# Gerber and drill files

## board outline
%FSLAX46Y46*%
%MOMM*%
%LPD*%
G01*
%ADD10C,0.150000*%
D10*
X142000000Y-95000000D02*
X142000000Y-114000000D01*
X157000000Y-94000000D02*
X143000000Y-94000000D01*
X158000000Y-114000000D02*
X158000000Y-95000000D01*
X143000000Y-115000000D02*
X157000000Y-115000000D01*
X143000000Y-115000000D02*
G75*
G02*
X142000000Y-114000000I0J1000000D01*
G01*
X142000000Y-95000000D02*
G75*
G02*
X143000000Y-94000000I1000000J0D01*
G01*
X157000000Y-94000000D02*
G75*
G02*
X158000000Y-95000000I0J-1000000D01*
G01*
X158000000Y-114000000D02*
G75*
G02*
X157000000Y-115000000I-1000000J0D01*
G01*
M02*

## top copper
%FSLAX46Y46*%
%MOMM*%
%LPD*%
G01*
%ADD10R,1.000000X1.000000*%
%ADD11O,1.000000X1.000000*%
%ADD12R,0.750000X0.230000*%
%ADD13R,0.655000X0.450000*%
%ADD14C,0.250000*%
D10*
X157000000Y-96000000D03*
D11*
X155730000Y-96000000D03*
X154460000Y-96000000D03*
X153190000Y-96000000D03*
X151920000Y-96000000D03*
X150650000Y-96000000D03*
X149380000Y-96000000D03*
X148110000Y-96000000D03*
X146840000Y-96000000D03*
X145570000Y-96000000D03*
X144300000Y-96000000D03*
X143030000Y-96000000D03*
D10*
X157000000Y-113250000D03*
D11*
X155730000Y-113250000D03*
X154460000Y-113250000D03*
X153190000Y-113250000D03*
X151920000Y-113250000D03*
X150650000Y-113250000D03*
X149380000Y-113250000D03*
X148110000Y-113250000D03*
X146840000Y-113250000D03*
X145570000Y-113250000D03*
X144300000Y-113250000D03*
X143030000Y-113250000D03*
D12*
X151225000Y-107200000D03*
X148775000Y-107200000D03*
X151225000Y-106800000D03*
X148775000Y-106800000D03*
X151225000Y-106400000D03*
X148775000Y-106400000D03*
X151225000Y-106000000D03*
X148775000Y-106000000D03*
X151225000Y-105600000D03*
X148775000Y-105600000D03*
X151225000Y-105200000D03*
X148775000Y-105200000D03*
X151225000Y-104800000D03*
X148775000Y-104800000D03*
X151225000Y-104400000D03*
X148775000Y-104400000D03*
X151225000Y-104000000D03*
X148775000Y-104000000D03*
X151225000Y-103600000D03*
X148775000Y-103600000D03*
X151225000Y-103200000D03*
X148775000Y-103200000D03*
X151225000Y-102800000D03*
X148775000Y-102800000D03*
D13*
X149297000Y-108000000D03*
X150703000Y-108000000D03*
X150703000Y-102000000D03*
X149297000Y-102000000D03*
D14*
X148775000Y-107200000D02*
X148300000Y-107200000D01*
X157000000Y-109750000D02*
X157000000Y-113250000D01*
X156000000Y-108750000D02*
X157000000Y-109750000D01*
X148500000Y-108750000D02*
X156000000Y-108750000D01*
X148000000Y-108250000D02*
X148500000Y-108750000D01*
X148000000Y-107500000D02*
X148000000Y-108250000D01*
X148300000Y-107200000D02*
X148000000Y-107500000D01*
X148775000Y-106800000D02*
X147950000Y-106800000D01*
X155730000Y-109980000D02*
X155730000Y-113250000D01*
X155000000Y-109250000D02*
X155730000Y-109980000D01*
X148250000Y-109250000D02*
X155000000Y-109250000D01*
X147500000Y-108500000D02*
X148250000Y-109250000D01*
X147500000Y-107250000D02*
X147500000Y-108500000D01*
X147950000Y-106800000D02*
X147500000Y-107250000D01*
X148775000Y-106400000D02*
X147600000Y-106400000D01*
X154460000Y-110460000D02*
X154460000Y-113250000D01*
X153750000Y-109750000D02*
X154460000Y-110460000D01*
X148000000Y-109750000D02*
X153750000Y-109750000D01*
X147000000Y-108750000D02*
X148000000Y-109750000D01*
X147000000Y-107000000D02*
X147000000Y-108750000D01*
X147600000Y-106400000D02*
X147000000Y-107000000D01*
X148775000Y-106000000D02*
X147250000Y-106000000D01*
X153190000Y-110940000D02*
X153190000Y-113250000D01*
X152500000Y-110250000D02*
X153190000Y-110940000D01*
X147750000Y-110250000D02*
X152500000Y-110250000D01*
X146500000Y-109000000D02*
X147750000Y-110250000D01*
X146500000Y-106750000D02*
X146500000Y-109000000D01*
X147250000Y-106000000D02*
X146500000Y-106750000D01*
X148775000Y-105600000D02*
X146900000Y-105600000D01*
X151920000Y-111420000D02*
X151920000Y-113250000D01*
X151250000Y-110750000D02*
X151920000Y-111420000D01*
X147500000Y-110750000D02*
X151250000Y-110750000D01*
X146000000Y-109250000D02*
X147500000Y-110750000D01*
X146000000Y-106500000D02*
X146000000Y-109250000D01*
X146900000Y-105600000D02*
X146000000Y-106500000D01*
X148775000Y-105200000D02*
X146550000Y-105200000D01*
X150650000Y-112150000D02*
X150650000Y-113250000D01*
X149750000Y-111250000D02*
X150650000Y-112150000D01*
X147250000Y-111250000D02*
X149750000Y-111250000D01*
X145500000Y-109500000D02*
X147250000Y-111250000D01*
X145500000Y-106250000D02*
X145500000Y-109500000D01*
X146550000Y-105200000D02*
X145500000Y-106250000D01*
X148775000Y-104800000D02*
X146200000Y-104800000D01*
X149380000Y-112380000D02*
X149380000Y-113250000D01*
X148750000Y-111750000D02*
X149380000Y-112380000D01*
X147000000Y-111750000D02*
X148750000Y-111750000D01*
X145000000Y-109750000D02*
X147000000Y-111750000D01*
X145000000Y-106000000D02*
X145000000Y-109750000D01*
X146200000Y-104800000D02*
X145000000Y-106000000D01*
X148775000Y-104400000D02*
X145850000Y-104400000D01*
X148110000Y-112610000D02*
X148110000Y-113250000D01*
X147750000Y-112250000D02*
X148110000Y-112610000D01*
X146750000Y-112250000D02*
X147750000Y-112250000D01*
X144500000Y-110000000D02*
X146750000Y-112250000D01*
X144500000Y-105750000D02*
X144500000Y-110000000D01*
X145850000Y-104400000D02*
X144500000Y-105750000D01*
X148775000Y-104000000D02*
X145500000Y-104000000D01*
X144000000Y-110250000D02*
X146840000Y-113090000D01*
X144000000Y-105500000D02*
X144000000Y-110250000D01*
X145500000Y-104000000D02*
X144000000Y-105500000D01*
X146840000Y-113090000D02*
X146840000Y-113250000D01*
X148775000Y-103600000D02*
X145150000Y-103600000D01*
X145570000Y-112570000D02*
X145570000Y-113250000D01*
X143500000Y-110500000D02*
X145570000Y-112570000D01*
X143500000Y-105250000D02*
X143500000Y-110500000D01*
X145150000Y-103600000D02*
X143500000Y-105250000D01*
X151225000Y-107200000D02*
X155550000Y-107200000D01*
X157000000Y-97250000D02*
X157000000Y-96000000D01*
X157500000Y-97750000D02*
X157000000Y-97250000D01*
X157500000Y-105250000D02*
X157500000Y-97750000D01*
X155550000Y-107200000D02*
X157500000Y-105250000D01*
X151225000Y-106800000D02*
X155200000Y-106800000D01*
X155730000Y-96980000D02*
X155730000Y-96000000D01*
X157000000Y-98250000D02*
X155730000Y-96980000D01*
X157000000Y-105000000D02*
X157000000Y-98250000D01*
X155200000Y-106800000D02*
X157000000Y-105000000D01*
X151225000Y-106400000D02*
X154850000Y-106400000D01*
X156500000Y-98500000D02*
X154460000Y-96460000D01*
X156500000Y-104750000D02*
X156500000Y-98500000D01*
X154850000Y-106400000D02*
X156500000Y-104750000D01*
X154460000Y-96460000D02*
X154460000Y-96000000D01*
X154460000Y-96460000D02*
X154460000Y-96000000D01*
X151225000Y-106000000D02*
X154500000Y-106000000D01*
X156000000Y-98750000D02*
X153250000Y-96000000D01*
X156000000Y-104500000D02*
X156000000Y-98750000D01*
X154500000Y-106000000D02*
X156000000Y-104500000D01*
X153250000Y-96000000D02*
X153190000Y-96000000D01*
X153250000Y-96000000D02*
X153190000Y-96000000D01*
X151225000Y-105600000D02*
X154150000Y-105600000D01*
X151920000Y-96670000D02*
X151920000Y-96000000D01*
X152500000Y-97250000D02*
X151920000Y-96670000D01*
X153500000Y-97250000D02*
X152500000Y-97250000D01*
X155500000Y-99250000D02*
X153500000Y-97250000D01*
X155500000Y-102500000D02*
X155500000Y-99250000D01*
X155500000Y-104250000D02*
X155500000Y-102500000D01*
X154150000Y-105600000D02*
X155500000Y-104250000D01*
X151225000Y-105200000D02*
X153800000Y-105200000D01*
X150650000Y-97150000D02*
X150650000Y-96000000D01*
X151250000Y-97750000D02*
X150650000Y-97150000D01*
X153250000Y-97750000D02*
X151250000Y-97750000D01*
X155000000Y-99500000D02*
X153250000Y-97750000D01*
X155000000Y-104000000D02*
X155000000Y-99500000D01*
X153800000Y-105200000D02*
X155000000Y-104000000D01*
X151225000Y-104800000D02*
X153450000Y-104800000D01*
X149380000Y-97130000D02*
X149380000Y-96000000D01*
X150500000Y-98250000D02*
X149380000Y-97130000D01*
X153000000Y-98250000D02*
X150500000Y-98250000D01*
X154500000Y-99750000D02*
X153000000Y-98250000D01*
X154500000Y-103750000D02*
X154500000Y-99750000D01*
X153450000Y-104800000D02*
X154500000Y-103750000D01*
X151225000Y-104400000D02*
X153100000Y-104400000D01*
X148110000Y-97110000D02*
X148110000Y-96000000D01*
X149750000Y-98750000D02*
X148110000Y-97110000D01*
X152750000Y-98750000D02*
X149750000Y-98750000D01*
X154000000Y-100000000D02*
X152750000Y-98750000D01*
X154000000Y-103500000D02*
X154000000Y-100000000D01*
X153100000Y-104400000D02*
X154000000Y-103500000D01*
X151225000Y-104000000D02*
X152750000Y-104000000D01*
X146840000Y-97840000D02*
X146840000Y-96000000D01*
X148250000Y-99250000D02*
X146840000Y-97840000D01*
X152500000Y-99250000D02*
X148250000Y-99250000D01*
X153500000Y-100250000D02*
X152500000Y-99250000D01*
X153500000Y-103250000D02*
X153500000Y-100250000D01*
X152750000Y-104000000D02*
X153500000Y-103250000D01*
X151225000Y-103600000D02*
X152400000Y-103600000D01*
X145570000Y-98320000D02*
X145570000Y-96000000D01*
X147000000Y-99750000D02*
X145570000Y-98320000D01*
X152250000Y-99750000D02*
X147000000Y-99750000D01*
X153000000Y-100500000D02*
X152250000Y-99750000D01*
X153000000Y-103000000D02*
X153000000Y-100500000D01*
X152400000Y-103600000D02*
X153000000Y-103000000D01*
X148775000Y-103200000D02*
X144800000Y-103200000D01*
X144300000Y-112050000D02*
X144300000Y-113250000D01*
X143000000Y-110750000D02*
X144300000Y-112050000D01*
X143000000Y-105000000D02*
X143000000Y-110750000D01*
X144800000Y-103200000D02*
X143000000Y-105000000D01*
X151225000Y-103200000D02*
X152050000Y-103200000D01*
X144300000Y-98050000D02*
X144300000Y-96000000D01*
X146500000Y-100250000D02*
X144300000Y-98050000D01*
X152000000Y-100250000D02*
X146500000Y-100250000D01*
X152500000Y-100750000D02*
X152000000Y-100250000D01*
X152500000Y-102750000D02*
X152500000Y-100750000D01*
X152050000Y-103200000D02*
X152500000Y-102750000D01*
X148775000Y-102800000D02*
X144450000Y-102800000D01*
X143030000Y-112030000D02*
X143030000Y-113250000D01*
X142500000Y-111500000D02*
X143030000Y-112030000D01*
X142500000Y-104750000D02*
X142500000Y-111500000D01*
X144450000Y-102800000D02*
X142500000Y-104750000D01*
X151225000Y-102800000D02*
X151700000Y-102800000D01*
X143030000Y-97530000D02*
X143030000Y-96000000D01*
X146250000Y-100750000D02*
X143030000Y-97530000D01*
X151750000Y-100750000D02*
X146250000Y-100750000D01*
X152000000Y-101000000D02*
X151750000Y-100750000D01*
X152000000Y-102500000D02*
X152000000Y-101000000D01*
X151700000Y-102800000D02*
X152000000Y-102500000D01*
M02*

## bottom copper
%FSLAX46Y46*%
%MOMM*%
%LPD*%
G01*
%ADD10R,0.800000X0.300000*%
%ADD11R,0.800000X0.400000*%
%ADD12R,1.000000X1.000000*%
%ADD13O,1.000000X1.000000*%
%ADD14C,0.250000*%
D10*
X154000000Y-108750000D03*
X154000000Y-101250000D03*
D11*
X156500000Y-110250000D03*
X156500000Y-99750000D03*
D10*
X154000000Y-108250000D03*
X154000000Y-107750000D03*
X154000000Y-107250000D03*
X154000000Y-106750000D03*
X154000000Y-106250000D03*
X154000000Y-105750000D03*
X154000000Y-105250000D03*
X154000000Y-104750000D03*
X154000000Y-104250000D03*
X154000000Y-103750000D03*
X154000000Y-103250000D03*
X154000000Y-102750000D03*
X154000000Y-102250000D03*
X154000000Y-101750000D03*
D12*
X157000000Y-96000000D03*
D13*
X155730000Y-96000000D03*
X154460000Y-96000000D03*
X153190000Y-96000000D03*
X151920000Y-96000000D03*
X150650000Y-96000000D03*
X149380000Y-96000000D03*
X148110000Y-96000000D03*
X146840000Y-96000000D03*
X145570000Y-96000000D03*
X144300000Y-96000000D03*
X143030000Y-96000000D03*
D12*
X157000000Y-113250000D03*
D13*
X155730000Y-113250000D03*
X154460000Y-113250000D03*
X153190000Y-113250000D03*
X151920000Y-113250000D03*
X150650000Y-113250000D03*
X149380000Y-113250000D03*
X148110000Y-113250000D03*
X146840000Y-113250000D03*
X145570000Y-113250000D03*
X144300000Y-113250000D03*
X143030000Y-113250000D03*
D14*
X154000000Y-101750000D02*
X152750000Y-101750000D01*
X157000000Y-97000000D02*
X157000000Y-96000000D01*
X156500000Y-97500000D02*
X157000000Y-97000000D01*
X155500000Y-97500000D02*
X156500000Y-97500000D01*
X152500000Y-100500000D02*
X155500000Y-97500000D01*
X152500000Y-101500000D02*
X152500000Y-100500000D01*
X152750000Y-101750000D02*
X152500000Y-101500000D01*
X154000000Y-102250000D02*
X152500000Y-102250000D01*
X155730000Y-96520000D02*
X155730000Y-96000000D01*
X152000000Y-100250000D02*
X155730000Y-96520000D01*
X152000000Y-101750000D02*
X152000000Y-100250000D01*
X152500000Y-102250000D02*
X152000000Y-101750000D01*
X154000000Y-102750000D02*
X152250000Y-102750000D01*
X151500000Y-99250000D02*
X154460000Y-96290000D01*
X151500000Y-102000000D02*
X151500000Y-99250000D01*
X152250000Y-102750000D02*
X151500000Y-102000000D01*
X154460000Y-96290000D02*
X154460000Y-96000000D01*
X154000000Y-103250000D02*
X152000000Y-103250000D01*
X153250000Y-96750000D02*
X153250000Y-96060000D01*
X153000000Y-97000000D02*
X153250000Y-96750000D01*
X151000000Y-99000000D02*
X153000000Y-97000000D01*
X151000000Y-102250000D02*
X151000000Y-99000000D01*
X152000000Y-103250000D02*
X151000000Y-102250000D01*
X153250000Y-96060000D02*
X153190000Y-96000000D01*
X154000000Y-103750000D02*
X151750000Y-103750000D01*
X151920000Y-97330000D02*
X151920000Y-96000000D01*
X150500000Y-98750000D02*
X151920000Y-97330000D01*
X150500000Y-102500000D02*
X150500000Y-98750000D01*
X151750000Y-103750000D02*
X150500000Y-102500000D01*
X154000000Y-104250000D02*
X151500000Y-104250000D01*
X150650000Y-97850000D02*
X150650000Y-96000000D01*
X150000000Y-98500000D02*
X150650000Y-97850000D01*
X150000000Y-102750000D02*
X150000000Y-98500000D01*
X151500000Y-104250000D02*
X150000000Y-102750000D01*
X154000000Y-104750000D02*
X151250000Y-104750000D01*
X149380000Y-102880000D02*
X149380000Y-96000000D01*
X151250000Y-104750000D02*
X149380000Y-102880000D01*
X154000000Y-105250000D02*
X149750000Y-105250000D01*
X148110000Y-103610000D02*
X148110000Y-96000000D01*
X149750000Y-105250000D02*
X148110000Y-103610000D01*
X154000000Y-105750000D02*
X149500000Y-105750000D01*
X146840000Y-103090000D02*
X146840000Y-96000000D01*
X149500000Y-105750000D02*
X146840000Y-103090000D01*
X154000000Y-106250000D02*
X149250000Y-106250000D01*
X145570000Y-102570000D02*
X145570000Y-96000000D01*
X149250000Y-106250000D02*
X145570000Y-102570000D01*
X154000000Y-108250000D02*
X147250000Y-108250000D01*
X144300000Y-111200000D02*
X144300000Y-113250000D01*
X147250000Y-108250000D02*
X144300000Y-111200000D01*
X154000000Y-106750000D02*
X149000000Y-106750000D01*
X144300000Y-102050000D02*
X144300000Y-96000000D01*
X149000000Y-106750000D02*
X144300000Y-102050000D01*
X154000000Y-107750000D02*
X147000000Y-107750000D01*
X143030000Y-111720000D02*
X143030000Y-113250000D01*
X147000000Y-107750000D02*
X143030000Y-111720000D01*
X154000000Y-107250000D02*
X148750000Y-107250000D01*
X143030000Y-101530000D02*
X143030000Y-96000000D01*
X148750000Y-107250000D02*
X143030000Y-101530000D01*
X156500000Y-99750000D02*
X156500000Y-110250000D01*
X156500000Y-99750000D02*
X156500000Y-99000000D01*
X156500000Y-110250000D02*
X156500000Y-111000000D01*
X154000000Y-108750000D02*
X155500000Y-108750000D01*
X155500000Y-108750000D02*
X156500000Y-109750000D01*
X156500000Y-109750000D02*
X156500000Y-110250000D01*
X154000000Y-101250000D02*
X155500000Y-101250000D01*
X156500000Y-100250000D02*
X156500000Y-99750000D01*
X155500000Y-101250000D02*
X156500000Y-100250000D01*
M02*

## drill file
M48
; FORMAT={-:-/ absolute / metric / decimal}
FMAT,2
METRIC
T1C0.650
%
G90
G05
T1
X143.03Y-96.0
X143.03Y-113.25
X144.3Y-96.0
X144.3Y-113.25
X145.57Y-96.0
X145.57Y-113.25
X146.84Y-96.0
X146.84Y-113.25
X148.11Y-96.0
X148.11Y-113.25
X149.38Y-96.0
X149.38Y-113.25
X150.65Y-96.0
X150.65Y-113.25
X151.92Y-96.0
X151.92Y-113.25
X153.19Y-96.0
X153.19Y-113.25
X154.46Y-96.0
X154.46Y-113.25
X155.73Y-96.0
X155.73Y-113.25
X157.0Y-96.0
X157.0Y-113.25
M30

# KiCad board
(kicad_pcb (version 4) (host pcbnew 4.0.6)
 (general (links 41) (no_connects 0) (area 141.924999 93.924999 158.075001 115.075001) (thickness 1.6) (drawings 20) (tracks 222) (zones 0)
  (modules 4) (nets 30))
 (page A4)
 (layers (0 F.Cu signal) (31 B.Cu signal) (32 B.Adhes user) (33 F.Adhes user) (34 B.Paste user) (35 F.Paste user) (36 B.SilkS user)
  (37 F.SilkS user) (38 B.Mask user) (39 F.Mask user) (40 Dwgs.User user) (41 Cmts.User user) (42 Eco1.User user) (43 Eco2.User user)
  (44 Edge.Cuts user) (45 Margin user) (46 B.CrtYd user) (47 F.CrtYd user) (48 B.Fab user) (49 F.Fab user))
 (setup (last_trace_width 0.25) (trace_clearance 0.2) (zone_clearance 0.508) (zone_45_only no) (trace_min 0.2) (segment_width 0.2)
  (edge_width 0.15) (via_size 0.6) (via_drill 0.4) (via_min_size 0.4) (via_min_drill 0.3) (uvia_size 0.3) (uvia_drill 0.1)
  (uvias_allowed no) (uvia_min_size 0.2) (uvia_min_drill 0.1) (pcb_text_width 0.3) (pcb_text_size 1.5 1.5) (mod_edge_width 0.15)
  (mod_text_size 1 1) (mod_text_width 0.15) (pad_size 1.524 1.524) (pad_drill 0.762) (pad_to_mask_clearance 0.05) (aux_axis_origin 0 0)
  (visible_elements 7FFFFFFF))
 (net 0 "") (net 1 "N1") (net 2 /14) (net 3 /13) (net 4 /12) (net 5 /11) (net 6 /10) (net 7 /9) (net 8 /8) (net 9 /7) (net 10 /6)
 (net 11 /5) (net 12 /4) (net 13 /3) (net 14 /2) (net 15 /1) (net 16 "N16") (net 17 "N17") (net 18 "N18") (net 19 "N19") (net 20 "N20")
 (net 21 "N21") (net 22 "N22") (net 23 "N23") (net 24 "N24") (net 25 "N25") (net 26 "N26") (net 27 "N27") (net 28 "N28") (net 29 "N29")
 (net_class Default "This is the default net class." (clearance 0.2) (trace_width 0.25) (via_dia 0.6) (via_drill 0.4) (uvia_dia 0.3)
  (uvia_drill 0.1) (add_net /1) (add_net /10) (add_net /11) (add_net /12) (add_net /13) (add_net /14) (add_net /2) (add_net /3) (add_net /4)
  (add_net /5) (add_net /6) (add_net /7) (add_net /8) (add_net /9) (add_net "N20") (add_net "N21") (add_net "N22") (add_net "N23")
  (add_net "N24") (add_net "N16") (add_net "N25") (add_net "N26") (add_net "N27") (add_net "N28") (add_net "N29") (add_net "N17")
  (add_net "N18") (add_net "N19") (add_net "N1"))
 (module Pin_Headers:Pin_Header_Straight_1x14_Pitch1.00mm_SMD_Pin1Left (layer B.Cu) (at 154 105 270)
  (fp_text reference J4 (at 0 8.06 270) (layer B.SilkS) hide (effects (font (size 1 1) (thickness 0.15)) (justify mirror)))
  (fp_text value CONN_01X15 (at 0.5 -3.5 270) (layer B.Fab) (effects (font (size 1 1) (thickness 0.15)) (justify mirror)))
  (pad 15 smd rect (at 3.75 0 270) (size 0.3 0.8) (layers B.Cu B.Paste B.Mask) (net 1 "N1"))
  (pad 15 smd rect (at -3.75 0 270) (size 0.3 0.8) (layers B.Cu B.Paste B.Mask) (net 1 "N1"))
  (pad 15 smd rect (at 5.25 -2.5 270) (size 0.4 0.8) (layers B.Cu B.Paste B.Mask) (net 1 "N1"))
  (pad 15 smd rect (at -5.25 -2.5 270) (size 0.4 0.8) (layers B.Cu B.Paste B.Mask) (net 1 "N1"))
  (pad 14 smd rect (at 3.25 0 270) (size 0.3 0.8) (layers B.Cu B.Paste B.Mask) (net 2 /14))
  (pad 13 smd rect (at 2.75 0 270) (size 0.3 0.8) (layers B.Cu B.Paste B.Mask) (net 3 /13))
  (pad 12 smd rect (at 2.25 0 270) (size 0.3 0.8) (layers B.Cu B.Paste B.Mask) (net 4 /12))
  (pad 11 smd rect (at 1.75 0 270) (size 0.3 0.8) (layers B.Cu B.Paste B.Mask) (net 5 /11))
  (pad 10 smd rect (at 1.25 0 270) (size 0.3 0.8) (layers B.Cu B.Paste B.Mask) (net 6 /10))
  (pad 9 smd rect (at 0.75 0 270) (size 0.3 0.8) (layers B.Cu B.Paste B.Mask) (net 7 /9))
  (pad 8 smd rect (at 0.25 0 270) (size 0.3 0.8) (layers B.Cu B.Paste B.Mask) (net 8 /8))
  (pad 7 smd rect (at -0.25 0 270) (size 0.3 0.8) (layers B.Cu B.Paste B.Mask) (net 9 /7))
  (pad 6 smd rect (at -0.75 0 270) (size 0.3 0.8) (layers B.Cu B.Paste B.Mask) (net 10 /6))
  (pad 5 smd rect (at -1.25 0 270) (size 0.3 0.8) (layers B.Cu B.Paste B.Mask) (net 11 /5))
  (pad 4 smd rect (at -1.75 0 270) (size 0.3 0.8) (layers B.Cu B.Paste B.Mask) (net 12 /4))
  (pad 3 smd rect (at -2.25 0 270) (size 0.3 0.8) (layers B.Cu B.Paste B.Mask) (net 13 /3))
  (pad 2 smd rect (at -2.75 0 270) (size 0.3 0.8) (layers B.Cu B.Paste B.Mask) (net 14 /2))
  (pad 1 smd rect (at -3.25 0 270) (size 0.3 0.8) (layers B.Cu B.Paste B.Mask) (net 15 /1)))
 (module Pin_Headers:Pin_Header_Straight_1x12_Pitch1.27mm (layer F.Cu) (at 157 96 270)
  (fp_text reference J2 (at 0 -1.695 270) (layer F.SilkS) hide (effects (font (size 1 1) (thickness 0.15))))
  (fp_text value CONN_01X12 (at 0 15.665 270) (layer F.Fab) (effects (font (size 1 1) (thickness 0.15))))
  (pad 1 thru_hole rect (at 0 0 270) (size 1 1) (drill 0.65) (layers *.Cu *.Mask) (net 15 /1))
  (pad 2 thru_hole oval (at 0 1.27 270) (size 1 1) (drill 0.65) (layers *.Cu *.Mask) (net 14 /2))
  (pad 3 thru_hole oval (at 0 2.54 270) (size 1 1) (drill 0.65) (layers *.Cu *.Mask) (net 13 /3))
  (pad 4 thru_hole oval (at 0 3.81 270) (size 1 1) (drill 0.65) (layers *.Cu *.Mask) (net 12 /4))
  (pad 5 thru_hole oval (at 0 5.08 270) (size 1 1) (drill 0.65) (layers *.Cu *.Mask) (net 11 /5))
  (pad 6 thru_hole oval (at 0 6.35 270) (size 1 1) (drill 0.65) (layers *.Cu *.Mask) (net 10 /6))
  (pad 7 thru_hole oval (at 0 7.62 270) (size 1 1) (drill 0.65) (layers *.Cu *.Mask) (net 9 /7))
  (pad 8 thru_hole oval (at 0 8.89 270) (size 1 1) (drill 0.65) (layers *.Cu *.Mask) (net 8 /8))
  (pad 9 thru_hole oval (at 0 10.16 270) (size 1 1) (drill 0.65) (layers *.Cu *.Mask) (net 7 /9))
  (pad 10 thru_hole oval (at 0 11.43 270) (size 1 1) (drill 0.65) (layers *.Cu *.Mask) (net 6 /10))
  (pad 11 thru_hole oval (at 0 12.7 270) (size 1 1) (drill 0.65) (layers *.Cu *.Mask) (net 5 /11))
  (pad 12 thru_hole oval (at 0 13.97 270) (size 1 1) (drill 0.65) (layers *.Cu *.Mask) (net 4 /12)))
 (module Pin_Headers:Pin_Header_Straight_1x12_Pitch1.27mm (layer F.Cu) (at 157 113.25 270)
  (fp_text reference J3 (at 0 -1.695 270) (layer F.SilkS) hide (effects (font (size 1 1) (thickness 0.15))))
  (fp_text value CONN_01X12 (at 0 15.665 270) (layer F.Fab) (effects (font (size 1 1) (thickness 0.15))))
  (pad 1 thru_hole rect (at 0 0 270) (size 1 1) (drill 0.65) (layers *.Cu *.Mask) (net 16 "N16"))
  (pad 2 thru_hole oval (at 0 1.27 270) (size 1 1) (drill 0.65) (layers *.Cu *.Mask) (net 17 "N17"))
  (pad 3 thru_hole oval (at 0 2.54 270) (size 1 1) (drill 0.65) (layers *.Cu *.Mask) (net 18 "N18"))
  (pad 4 thru_hole oval (at 0 3.81 270) (size 1 1) (drill 0.65) (layers *.Cu *.Mask) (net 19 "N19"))
  (pad 5 thru_hole oval (at 0 5.08 270) (size 1 1) (drill 0.65) (layers *.Cu *.Mask) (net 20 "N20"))
  (pad 6 thru_hole oval (at 0 6.35 270) (size 1 1) (drill 0.65) (layers *.Cu *.Mask) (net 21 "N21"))
  (pad 7 thru_hole oval (at 0 7.62 270) (size 1 1) (drill 0.65) (layers *.Cu *.Mask) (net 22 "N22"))
  (pad 8 thru_hole oval (at 0 8.89 270) (size 1 1) (drill 0.65) (layers *.Cu *.Mask) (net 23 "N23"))
  (pad 9 thru_hole oval (at 0 10.16 270) (size 1 1) (drill 0.65) (layers *.Cu *.Mask) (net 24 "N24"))
  (pad 10 thru_hole oval (at 0 11.43 270) (size 1 1) (drill 0.65) (layers *.Cu *.Mask) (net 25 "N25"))
  (pad 11 thru_hole oval (at 0 12.7 270) (size 1 1) (drill 0.65) (layers *.Cu *.Mask) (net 2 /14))
  (pad 12 thru_hole oval (at 0 13.97 270) (size 1 1) (drill 0.65) (layers *.Cu *.Mask) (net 3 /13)))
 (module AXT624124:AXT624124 (layer F.Cu) (at 150 105 90)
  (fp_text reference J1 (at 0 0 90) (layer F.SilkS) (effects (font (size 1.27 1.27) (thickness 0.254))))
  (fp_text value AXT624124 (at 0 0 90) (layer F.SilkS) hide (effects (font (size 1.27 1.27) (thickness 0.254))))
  (pad 1 smd rect (at -2.2 1.225 90) (size 0.23 0.75) (layers F.Cu F.Paste F.Mask) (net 15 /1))
  (pad 2 smd rect (at -2.2 -1.225 90) (size 0.23 0.75) (layers F.Cu F.Paste F.Mask) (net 16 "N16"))
  (pad 3 smd rect (at -1.8 1.225 90) (size 0.23 0.75) (layers F.Cu F.Paste F.Mask) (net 14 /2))
  (pad 4 smd rect (at -1.8 -1.225 90) (size 0.23 0.75) (layers F.Cu F.Paste F.Mask) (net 17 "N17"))
  (pad 5 smd rect (at -1.4 1.225 90) (size 0.23 0.75) (layers F.Cu F.Paste F.Mask) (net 13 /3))
  (pad 6 smd rect (at -1.4 -1.225 90) (size 0.23 0.75) (layers F.Cu F.Paste F.Mask) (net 18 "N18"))
  (pad 7 smd rect (at -1 1.225 90) (size 0.23 0.75) (layers F.Cu F.Paste F.Mask) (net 12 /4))
  (pad 8 smd rect (at -1 -1.225 90) (size 0.23 0.75) (layers F.Cu F.Paste F.Mask) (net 19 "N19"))
  (pad 9 smd rect (at -0.6 1.225 90) (size 0.23 0.75) (layers F.Cu F.Paste F.Mask) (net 11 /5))
  (pad 10 smd rect (at -0.6 -1.225 90) (size 0.23 0.75) (layers F.Cu F.Paste F.Mask) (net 20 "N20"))
  (pad 11 smd rect (at -0.2 1.225 90) (size 0.23 0.75) (layers F.Cu F.Paste F.Mask) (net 10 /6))
  (pad 12 smd rect (at -0.2 -1.225 90) (size 0.23 0.75) (layers F.Cu F.Paste F.Mask) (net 21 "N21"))
  (pad 13 smd rect (at 0.2 1.225 90) (size 0.23 0.75) (layers F.Cu F.Paste F.Mask) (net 9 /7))
  (pad 14 smd rect (at 0.2 -1.225 90) (size 0.23 0.75) (layers F.Cu F.Paste F.Mask) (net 22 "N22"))
  (pad 15 smd rect (at 0.6 1.225 90) (size 0.23 0.75) (layers F.Cu F.Paste F.Mask) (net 8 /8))
  (pad 16 smd rect (at 0.6 -1.225 90) (size 0.23 0.75) (layers F.Cu F.Paste F.Mask) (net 23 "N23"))
  (pad 17 smd rect (at 1 1.225 90) (size 0.23 0.75) (layers F.Cu F.Paste F.Mask) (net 7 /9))
  (pad 18 smd rect (at 1 -1.225 90) (size 0.23 0.75) (layers F.Cu F.Paste F.Mask) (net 24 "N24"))
  (pad 19 smd rect (at 1.4 1.225 90) (size 0.23 0.75) (layers F.Cu F.Paste F.Mask) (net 6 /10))
  (pad 20 smd rect (at 1.4 -1.225 90) (size 0.23 0.75) (layers F.Cu F.Paste F.Mask) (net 25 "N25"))
  (pad 21 smd rect (at 1.8 1.225 90) (size 0.23 0.75) (layers F.Cu F.Paste F.Mask) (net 5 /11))
  (pad 22 smd rect (at 1.8 -1.225 90) (size 0.23 0.75) (layers F.Cu F.Paste F.Mask) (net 2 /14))
  (pad 23 smd rect (at 2.2 1.225 90) (size 0.23 0.75) (layers F.Cu F.Paste F.Mask) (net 4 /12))
  (pad 24 smd rect (at 2.2 -1.225 90) (size 0.23 0.75) (layers F.Cu F.Paste F.Mask) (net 3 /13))
  (pad 25 smd rect (at -3 -0.703 90) (size 0.45 0.655) (layers F.Cu F.Paste F.Mask) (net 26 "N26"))
  (pad 26 smd rect (at -3 0.703 90) (size 0.45 0.655) (layers F.Cu F.Paste F.Mask) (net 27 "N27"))
  (pad 27 smd rect (at 3 0.703 90) (size 0.45 0.655) (layers F.Cu F.Paste F.Mask) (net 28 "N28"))
  (pad 28 smd rect (at 3 -0.703 90) (size 0.45 0.655) (layers F.Cu F.Paste F.Mask) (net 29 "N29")))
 (gr_line (start 142 95) (end 142 114) (angle 90) (layer Edge.Cuts) (width 0.15))
 (gr_line (start 157 94) (end 143 94) (angle 90) (layer Edge.Cuts) (width 0.15))
 (gr_line (start 158 114) (end 158 95) (angle 90) (layer Edge.Cuts) (width 0.15))
 (gr_line (start 143 115) (end 157 115) (angle 90) (layer Edge.Cuts) (width 0.15))
 (gr_arc (start 143 114) (end 143 115) (angle 90) (layer Edge.Cuts) (width 0.15))
 (gr_arc (start 143 95) (end 142 95) (angle 90) (layer Edge.Cuts) (width 0.15))
 (gr_arc (start 157 95) (end 157 94) (angle 90) (layer Edge.Cuts) (width 0.15))
 (gr_arc (start 157 114) (end 158 114) (angle 90) (layer Edge.Cuts) (width 0.15))
 (segment (start 148.775 107.2) (end 148.3 107.2) (width 0.25) (layer F.Cu) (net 16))
 (segment (start 157 109.75) (end 157 113.25) (width 0.25) (layer F.Cu) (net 16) (status 20))
 (segment (start 156 108.75) (end 157 109.75) (width 0.25) (layer F.Cu) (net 16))
 (segment (start 148.5 108.75) (end 156 108.75) (width 0.25) (layer F.Cu) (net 16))
 (segment (start 148 108.25) (end 148.5 108.75) (width 0.25) (layer F.Cu) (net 16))
 (segment (start 148 107.5) (end 148 108.25) (width 0.25) (layer F.Cu) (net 16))
 (segment (start 148.3 107.2) (end 148 107.5) (width 0.25) (layer F.Cu) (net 16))
 (segment (start 148.775 106.8) (end 147.95 106.8) (width 0.25) (layer F.Cu) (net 17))
 (segment (start 155.73 109.98) (end 155.73 113.25) (width 0.25) (layer F.Cu) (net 17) (status 20))
 (segment (start 155 109.25) (end 155.73 109.98) (width 0.25) (layer F.Cu) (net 17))
 (segment (start 148.25 109.25) (end 155 109.25) (width 0.25) (layer F.Cu) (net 17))
 (segment (start 147.5 108.5) (end 148.25 109.25) (width 0.25) (layer F.Cu) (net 17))
 (segment (start 147.5 107.25) (end 147.5 108.5) (width 0.25) (layer F.Cu) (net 17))
 (segment (start 147.95 106.8) (end 147.5 107.25) (width 0.25) (layer F.Cu) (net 17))
 (segment (start 148.775 106.4) (end 147.6 106.4) (width 0.25) (layer F.Cu) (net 18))
 (segment (start 154.46 110.46) (end 154.46 113.25) (width 0.25) (layer F.Cu) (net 18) (status 20))
 (segment (start 153.75 109.75) (end 154.46 110.46) (width 0.25) (layer F.Cu) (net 18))
 (segment (start 148 109.75) (end 153.75 109.75) (width 0.25) (layer F.Cu) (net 18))
 (segment (start 147 108.75) (end 148 109.75) (width 0.25) (layer F.Cu) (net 18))
 (segment (start 147 107) (end 147 108.75) (width 0.25) (layer F.Cu) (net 18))
 (segment (start 147.6 106.4) (end 147 107) (width 0.25) (layer F.Cu) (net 18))
 (segment (start 148.775 106) (end 147.25 106) (width 0.25) (layer F.Cu) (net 19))
 (segment (start 153.19 110.94) (end 153.19 113.25) (width 0.25) (layer F.Cu) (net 19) (status 20))
 (segment (start 152.5 110.25) (end 153.19 110.94) (width 0.25) (layer F.Cu) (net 19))
 (segment (start 147.75 110.25) (end 152.5 110.25) (width 0.25) (layer F.Cu) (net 19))
 (segment (start 146.5 109) (end 147.75 110.25) (width 0.25) (layer F.Cu) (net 19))
 (segment (start 146.5 106.75) (end 146.5 109) (width 0.25) (layer F.Cu) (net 19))
 (segment (start 147.25 106) (end 146.5 106.75) (width 0.25) (layer F.Cu) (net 19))
 (segment (start 148.775 105.6) (end 146.9 105.6) (width 0.25) (layer F.Cu) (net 20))
 (segment (start 151.92 111.42) (end 151.92 113.25) (width 0.25) (layer F.Cu) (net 20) (status 20))
 (segment (start 151.25 110.75) (end 151.92 111.42) (width 0.25) (layer F.Cu) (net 20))
 (segment (start 147.5 110.75) (end 151.25 110.75) (width 0.25) (layer F.Cu) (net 20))
 (segment (start 146 109.25) (end 147.5 110.75) (width 0.25) (layer F.Cu) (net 20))
 (segment (start 146 106.5) (end 146 109.25) (width 0.25) (layer F.Cu) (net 20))
 (segment (start 146.9 105.6) (end 146 106.5) (width 0.25) (layer F.Cu) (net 20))
 (segment (start 148.775 105.2) (end 146.55 105.2) (width 0.25) (layer F.Cu) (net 21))
 (segment (start 150.65 112.15) (end 150.65 113.25) (width 0.25) (layer F.Cu) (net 21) (status 20))
 (segment (start 149.75 111.25) (end 150.65 112.15) (width 0.25) (layer F.Cu) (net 21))
 (segment (start 147.25 111.25) (end 149.75 111.25) (width 0.25) (layer F.Cu) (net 21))
 (segment (start 145.5 109.5) (end 147.25 111.25) (width 0.25) (layer F.Cu) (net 21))
 (segment (start 145.5 106.25) (end 145.5 109.5) (width 0.25) (layer F.Cu) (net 21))
 (segment (start 146.55 105.2) (end 145.5 106.25) (width 0.25) (layer F.Cu) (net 21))
 (segment (start 148.775 104.8) (end 146.2 104.8) (width 0.25) (layer F.Cu) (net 22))
 (segment (start 149.38 112.38) (end 149.38 113.25) (width 0.25) (layer F.Cu) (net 22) (status 20))
 (segment (start 148.75 111.75) (end 149.38 112.38) (width 0.25) (layer F.Cu) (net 22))
 (segment (start 147 111.75) (end 148.75 111.75) (width 0.25) (layer F.Cu) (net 22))
 (segment (start 145 109.75) (end 147 111.75) (width 0.25) (layer F.Cu) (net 22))
 (segment (start 145 106) (end 145 109.75) (width 0.25) (layer F.Cu) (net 22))
 (segment (start 146.2 104.8) (end 145 106) (width 0.25) (layer F.Cu) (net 22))
 (segment (start 148.775 104.4) (end 145.85 104.4) (width 0.25) (layer F.Cu) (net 23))
 (segment (start 148.11 112.61) (end 148.11 113.25) (width 0.25) (layer F.Cu) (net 23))
 (segment (start 147.75 112.25) (end 148.11 112.61) (width 0.25) (layer F.Cu) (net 23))
 (segment (start 146.75 112.25) (end 147.75 112.25) (width 0.25) (layer F.Cu) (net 23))
 (segment (start 144.5 110) (end 146.75 112.25) (width 0.25) (layer F.Cu) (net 23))
 (segment (start 144.5 105.75) (end 144.5 110) (width 0.25) (layer F.Cu) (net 23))
 (segment (start 145.85 104.4) (end 144.5 105.75) (width 0.25) (layer F.Cu) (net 23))
 (segment (start 148.775 104) (end 145.5 104) (width 0.25) (layer F.Cu) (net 24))
 (segment (start 144 110.25) (end 146.84 113.09) (width 0.25) (layer F.Cu) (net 24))
 (segment (start 144 105.5) (end 144 110.25) (width 0.25) (layer F.Cu) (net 24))
 (segment (start 145.5 104) (end 144 105.5) (width 0.25) (layer F.Cu) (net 24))
 (segment (start 146.84 113.09) (end 146.84 113.25) (width 0.25) (layer F.Cu) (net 24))
 (segment (start 148.775 103.6) (end 145.15 103.6) (width 0.25) (layer F.Cu) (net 25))
 (segment (start 145.57 112.57) (end 145.57 113.25) (width 0.25) (layer F.Cu) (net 25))
 (segment (start 143.5 110.5) (end 145.57 112.57) (width 0.25) (layer F.Cu) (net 25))
 (segment (start 143.5 105.25) (end 143.5 110.5) (width 0.25) (layer F.Cu) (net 25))
 (segment (start 145.15 103.6) (end 143.5 105.25) (width 0.25) (layer F.Cu) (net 25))
 (segment (start 151.225 107.2) (end 155.55 107.2) (width 0.25) (layer F.Cu) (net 15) (status 400000))
 (segment (start 157 97.25) (end 157 96) (width 0.25) (layer F.Cu) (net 15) (status 800000))
 (segment (start 157.5 97.75) (end 157 97.25) (width 0.25) (layer F.Cu) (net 15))
 (segment (start 157.5 105.25) (end 157.5 97.75) (width 0.25) (layer F.Cu) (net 15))
 (segment (start 155.55 107.2) (end 157.5 105.25) (width 0.25) (layer F.Cu) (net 15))
 (segment (start 154 101.75) (end 152.75 101.75) (width 0.25) (layer B.Cu) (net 15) (status 400000))
 (segment (start 157 97) (end 157 96) (width 0.25) (layer B.Cu) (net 15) (status 800000))
 (segment (start 156.5 97.5) (end 157 97) (width 0.25) (layer B.Cu) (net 15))
 (segment (start 155.5 97.5) (end 156.5 97.5) (width 0.25) (layer B.Cu) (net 15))
 (segment (start 152.5 100.5) (end 155.5 97.5) (width 0.25) (layer B.Cu) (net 15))
 (segment (start 152.5 101.5) (end 152.5 100.5) (width 0.25) (layer B.Cu) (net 15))
 (segment (start 152.75 101.75) (end 152.5 101.5) (width 0.25) (layer B.Cu) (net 15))
 (segment (start 151.225 106.8) (end 155.2 106.8) (width 0.25) (layer F.Cu) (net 14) (status 400000))
 (segment (start 155.73 96.98) (end 155.73 96) (width 0.25) (layer F.Cu) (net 14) (status 800000))
 (segment (start 157 98.25) (end 155.73 96.98) (width 0.25) (layer F.Cu) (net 14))
 (segment (start 157 105) (end 157 98.25) (width 0.25) (layer F.Cu) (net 14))
 (segment (start 155.2 106.8) (end 157 105) (width 0.25) (layer F.Cu) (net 14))
 (segment (start 154 102.25) (end 152.5 102.25) (width 0.25) (layer B.Cu) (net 14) (status 400000))
 (segment (start 155.73 96.52) (end 155.73 96) (width 0.25) (layer B.Cu) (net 14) (status 800000))
 (segment (start 152 100.25) (end 155.73 96.52) (width 0.25) (layer B.Cu) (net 14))
 (segment (start 152 101.75) (end 152 100.25) (width 0.25) (layer B.Cu) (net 14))
 (segment (start 152.5 102.25) (end 152 101.75) (width 0.25) (layer B.Cu) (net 14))
 (segment (start 151.225 106.4) (end 154.85 106.4) (width 0.25) (layer F.Cu) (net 13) (status 400000))
 (segment (start 156.5 98.5) (end 154.46 96.46) (width 0.25) (layer F.Cu) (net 13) (status 800000))
 (segment (start 156.5 104.75) (end 156.5 98.5) (width 0.25) (layer F.Cu) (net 13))
 (segment (start 154.85 106.4) (end 156.5 104.75) (width 0.25) (layer F.Cu) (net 13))
 (segment (start 154.46 96.46) (end 154.46 96) (width 0.25) (layer F.Cu) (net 13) (status C00000))
 (segment (start 154 102.75) (end 152.25 102.75) (width 0.25) (layer B.Cu) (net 13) (status 400000))
 (segment (start 151.5 99.25) (end 154.46 96.29) (width 0.25) (layer B.Cu) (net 13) (status 800000))
 (segment (start 151.5 102) (end 151.5 99.25) (width 0.25) (layer B.Cu) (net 13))
 (segment (start 152.25 102.75) (end 151.5 102) (width 0.25) (layer B.Cu) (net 13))
 (segment (start 154.46 96.29) (end 154.46 96) (width 0.25) (layer B.Cu) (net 13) (status C00000))
 (segment (start 154.46 96.46) (end 154.46 96) (width 0.25) (layer F.Cu) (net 13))
 (segment (start 151.225 106) (end 154.5 106) (width 0.25) (layer F.Cu) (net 12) (status 400000))
 (segment (start 156 98.75) (end 153.25 96) (width 0.25) (layer F.Cu) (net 12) (status 800000))
 (segment (start 156 104.5) (end 156 98.75) (width 0.25) (layer F.Cu) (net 12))
 (segment (start 154.5 106) (end 156 104.5) (width 0.25) (layer F.Cu) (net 12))
 (segment (start 153.25 96) (end 153.19 96) (width 0.25) (layer F.Cu) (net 12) (status C00000))
 (segment (start 154 103.25) (end 152 103.25) (width 0.25) (layer B.Cu) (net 12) (status 400000))
 (segment (start 153.25 96.75) (end 153.25 96.06) (width 0.25) (layer B.Cu) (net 12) (status 800000))
 (segment (start 153 97) (end 153.25 96.75) (width 0.25) (layer B.Cu) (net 12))
 (segment (start 151 99) (end 153 97) (width 0.25) (layer B.Cu) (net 12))
 (segment (start 151 102.25) (end 151 99) (width 0.25) (layer B.Cu) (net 12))
 (segment (start 152 103.25) (end 151 102.25) (width 0.25) (layer B.Cu) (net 12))
 (segment (start 153.25 96.06) (end 153.19 96) (width 0.25) (layer B.Cu) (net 12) (status C00000))
 (segment (start 153.25 96) (end 153.19 96) (width 0.25) (layer F.Cu) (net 12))
 (segment (start 151.225 105.6) (end 154.15 105.6) (width 0.25) (layer F.Cu) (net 11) (status 400000))
 (segment (start 151.92 96.67) (end 151.92 96) (width 0.25) (layer F.Cu) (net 11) (status 800000))
 (segment (start 152.5 97.25) (end 151.92 96.67) (width 0.25) (layer F.Cu) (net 11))
 (segment (start 153.5 97.25) (end 152.5 97.25) (width 0.25) (layer F.Cu) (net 11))
 (segment (start 155.5 99.25) (end 153.5 97.25) (width 0.25) (layer F.Cu) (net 11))
 (segment (start 155.5 102.5) (end 155.5 99.25) (width 0.25) (layer F.Cu) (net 11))
 (segment (start 155.5 104.25) (end 155.5 102.5) (width 0.25) (layer F.Cu) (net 11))
 (segment (start 154.15 105.6) (end 155.5 104.25) (width 0.25) (layer F.Cu) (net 11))
 (segment (start 154 103.75) (end 151.75 103.75) (width 0.25) (layer B.Cu) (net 11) (status 400000))
 (segment (start 151.92 97.33) (end 151.92 96) (width 0.25) (layer B.Cu) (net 11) (status 800000))
 (segment (start 150.5 98.75) (end 151.92 97.33) (width 0.25) (layer B.Cu) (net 11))
 (segment (start 150.5 102.5) (end 150.5 98.75) (width 0.25) (layer B.Cu) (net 11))
 (segment (start 151.75 103.75) (end 150.5 102.5) (width 0.25) (layer B.Cu) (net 11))
 (segment (start 151.225 105.2) (end 153.8 105.2) (width 0.25) (layer F.Cu) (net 10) (status 400000))
 (segment (start 150.65 97.15) (end 150.65 96) (width 0.25) (layer F.Cu) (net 10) (status 800000))
 (segment (start 151.25 97.75) (end 150.65 97.15) (width 0.25) (layer F.Cu) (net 10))
 (segment (start 153.25 97.75) (end 151.25 97.75) (width 0.25) (layer F.Cu) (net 10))
 (segment (start 155 99.5) (end 153.25 97.75) (width 0.25) (layer F.Cu) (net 10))
 (segment (start 155 104) (end 155 99.5) (width 0.25) (layer F.Cu) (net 10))
 (segment (start 153.8 105.2) (end 155 104) (width 0.25) (layer F.Cu) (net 10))
 (segment (start 154 104.25) (end 151.5 104.25) (width 0.25) (layer B.Cu) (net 10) (status 400000))
 (segment (start 150.65 97.85) (end 150.65 96) (width 0.25) (layer B.Cu) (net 10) (status 800000))
 (segment (start 150 98.5) (end 150.65 97.85) (width 0.25) (layer B.Cu) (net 10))
 (segment (start 150 102.75) (end 150 98.5) (width 0.25) (layer B.Cu) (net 10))
 (segment (start 151.5 104.25) (end 150 102.75) (width 0.25) (layer B.Cu) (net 10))
 (segment (start 151.225 104.8) (end 153.45 104.8) (width 0.25) (layer F.Cu) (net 9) (status 400000))
 (segment (start 149.38 97.13) (end 149.38 96) (width 0.25) (layer F.Cu) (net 9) (status 800000))
 (segment (start 150.5 98.25) (end 149.38 97.13) (width 0.25) (layer F.Cu) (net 9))
 (segment (start 153 98.25) (end 150.5 98.25) (width 0.25) (layer F.Cu) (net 9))
 (segment (start 154.5 99.75) (end 153 98.25) (width 0.25) (layer F.Cu) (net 9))
 (segment (start 154.5 103.75) (end 154.5 99.75) (width 0.25) (layer F.Cu) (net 9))
 (segment (start 153.45 104.8) (end 154.5 103.75) (width 0.25) (layer F.Cu) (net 9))
 (segment (start 154 104.75) (end 151.25 104.75) (width 0.25) (layer B.Cu) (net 9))
 (segment (start 149.38 102.88) (end 149.38 96) (width 0.25) (layer B.Cu) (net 9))
 (segment (start 151.25 104.75) (end 149.38 102.88) (width 0.25) (layer B.Cu) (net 9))
 (segment (start 151.225 104.4) (end 153.1 104.4) (width 0.25) (layer F.Cu) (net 8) (status 400000))
 (segment (start 148.11 97.11) (end 148.11 96) (width 0.25) (layer F.Cu) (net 8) (status 800000))
 (segment (start 149.75 98.75) (end 148.11 97.11) (width 0.25) (layer F.Cu) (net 8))
 (segment (start 152.75 98.75) (end 149.75 98.75) (width 0.25) (layer F.Cu) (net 8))
 (segment (start 154 100) (end 152.75 98.75) (width 0.25) (layer F.Cu) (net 8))
 (segment (start 154 103.5) (end 154 100) (width 0.25) (layer F.Cu) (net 8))
 (segment (start 153.1 104.4) (end 154 103.5) (width 0.25) (layer F.Cu) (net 8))
 (segment (start 154 105.25) (end 149.75 105.25) (width 0.25) (layer B.Cu) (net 8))
 (segment (start 148.11 103.61) (end 148.11 96) (width 0.25) (layer B.Cu) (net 8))
 (segment (start 149.75 105.25) (end 148.11 103.61) (width 0.25) (layer B.Cu) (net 8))
 (segment (start 151.225 104) (end 152.75 104) (width 0.25) (layer F.Cu) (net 7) (status 400000))
 (segment (start 146.84 97.84) (end 146.84 96) (width 0.25) (layer F.Cu) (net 7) (status 800000))
 (segment (start 148.25 99.25) (end 146.84 97.84) (width 0.25) (layer F.Cu) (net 7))
 (segment (start 152.5 99.25) (end 148.25 99.25) (width 0.25) (layer F.Cu) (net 7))
 (segment (start 153.5 100.25) (end 152.5 99.25) (width 0.25) (layer F.Cu) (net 7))
 (segment (start 153.5 103.25) (end 153.5 100.25) (width 0.25) (layer F.Cu) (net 7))
 (segment (start 152.75 104) (end 153.5 103.25) (width 0.25) (layer F.Cu) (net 7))
 (segment (start 154 105.75) (end 149.5 105.75) (width 0.25) (layer B.Cu) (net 7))
 (segment (start 146.84 103.09) (end 146.84 96) (width 0.25) (layer B.Cu) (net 7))
 (segment (start 149.5 105.75) (end 146.84 103.09) (width 0.25) (layer B.Cu) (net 7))
 (segment (start 151.225 103.6) (end 152.4 103.6) (width 0.25) (layer F.Cu) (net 6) (status 400000))
 (segment (start 145.57 98.32) (end 145.57 96) (width 0.25) (layer F.Cu) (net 6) (status 800000))
 (segment (start 147 99.75) (end 145.57 98.32) (width 0.25) (layer F.Cu) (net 6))
 (segment (start 152.25 99.75) (end 147 99.75) (width 0.25) (layer F.Cu) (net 6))
 (segment (start 153 100.5) (end 152.25 99.75) (width 0.25) (layer F.Cu) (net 6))
 (segment (start 153 103) (end 153 100.5) (width 0.25) (layer F.Cu) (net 6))
 (segment (start 152.4 103.6) (end 153 103) (width 0.25) (layer F.Cu) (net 6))
 (segment (start 154 106.25) (end 149.25 106.25) (width 0.25) (layer B.Cu) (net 6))
 (segment (start 145.57 102.57) (end 145.57 96) (width 0.25) (layer B.Cu) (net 6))
 (segment (start 149.25 106.25) (end 145.57 102.57) (width 0.25) (layer B.Cu) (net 6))
 (segment (start 154 108.25) (end 147.25 108.25) (width 0.25) (layer B.Cu) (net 2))
 (segment (start 144.3 111.2) (end 144.3 113.25) (width 0.25) (layer B.Cu) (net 2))
 (segment (start 147.25 108.25) (end 144.3 111.2) (width 0.25) (layer B.Cu) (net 2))
 (segment (start 148.775 103.2) (end 144.8 103.2) (width 0.25) (layer F.Cu) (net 2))
 (segment (start 144.3 112.05) (end 144.3 113.25) (width 0.25) (layer F.Cu) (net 2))
 (segment (start 143 110.75) (end 144.3 112.05) (width 0.25) (layer F.Cu) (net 2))
 (segment (start 143 105) (end 143 110.75) (width 0.25) (layer F.Cu) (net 2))
 (segment (start 144.8 103.2) (end 143 105) (width 0.25) (layer F.Cu) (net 2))
 (segment (start 151.225 103.2) (end 152.05 103.2) (width 0.25) (layer F.Cu) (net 5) (status 400000))
 (segment (start 144.3 98.05) (end 144.3 96) (width 0.25) (layer F.Cu) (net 5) (status 800000))
 (segment (start 146.5 100.25) (end 144.3 98.05) (width 0.25) (layer F.Cu) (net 5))
 (segment (start 152 100.25) (end 146.5 100.25) (width 0.25) (layer F.Cu) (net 5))
 (segment (start 152.5 100.75) (end 152 100.25) (width 0.25) (layer F.Cu) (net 5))
 (segment (start 152.5 102.75) (end 152.5 100.75) (width 0.25) (layer F.Cu) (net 5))
 (segment (start 152.05 103.2) (end 152.5 102.75) (width 0.25) (layer F.Cu) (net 5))
 (segment (start 154 106.75) (end 149 106.75) (width 0.25) (layer B.Cu) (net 5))
 (segment (start 144.3 102.05) (end 144.3 96) (width 0.25) (layer B.Cu) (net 5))
 (segment (start 149 106.75) (end 144.3 102.05) (width 0.25) (layer B.Cu) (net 5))
 (segment (start 154 107.75) (end 147 107.75) (width 0.25) (layer B.Cu) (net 3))
 (segment (start 143.03 111.72) (end 143.03 113.25) (width 0.25) (layer B.Cu) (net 3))
 (segment (start 147 107.75) (end 143.03 111.72) (width 0.25) (layer B.Cu) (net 3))
 (segment (start 148.775 102.8) (end 144.45 102.8) (width 0.25) (layer F.Cu) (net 3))
 (segment (start 143.03 112.03) (end 143.03 113.25) (width 0.25) (layer F.Cu) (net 3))
 (segment (start 142.5 111.5) (end 143.03 112.03) (width 0.25) (layer F.Cu) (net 3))
 (segment (start 142.5 104.75) (end 142.5 111.5) (width 0.25) (layer F.Cu) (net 3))
 (segment (start 144.45 102.8) (end 142.5 104.75) (width 0.25) (layer F.Cu) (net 3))
 (segment (start 151.225 102.8) (end 151.7 102.8) (width 0.25) (layer F.Cu) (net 4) (status 400000))
 (segment (start 143.03 97.53) (end 143.03 96) (width 0.25) (layer F.Cu) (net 4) (status 800000))
 (segment (start 146.25 100.75) (end 143.03 97.53) (width 0.25) (layer F.Cu) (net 4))
 (segment (start 151.75 100.75) (end 146.25 100.75) (width 0.25) (layer F.Cu) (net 4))
 (segment (start 152 101) (end 151.75 100.75) (width 0.25) (layer F.Cu) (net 4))
 (segment (start 152 102.5) (end 152 101) (width 0.25) (layer F.Cu) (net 4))
 (segment (start 151.7 102.8) (end 152 102.5) (width 0.25) (layer F.Cu) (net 4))
 (segment (start 154 107.25) (end 148.75 107.25) (width 0.25) (layer B.Cu) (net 4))
 (segment (start 143.03 101.53) (end 143.03 96) (width 0.25) (layer B.Cu) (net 4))
 (segment (start 148.75 107.25) (end 143.03 101.53) (width 0.25) (layer B.Cu) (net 4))
 (segment (start 156.5 99.75) (end 156.5 110.25) (width 0.25) (layer B.Cu) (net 1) (status C00000))
 (segment (start 156.5 99.75) (end 156.5 99) (width 0.25) (layer B.Cu) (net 1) (status 400000))
 (segment (start 156.5 110.25) (end 156.5 111) (width 0.25) (layer B.Cu) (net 1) (status 400000))
 (segment (start 154 108.75) (end 155.5 108.75) (width 0.25) (layer B.Cu) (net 1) (status 400000))
 (segment (start 155.5 108.75) (end 156.5 109.75) (width 0.25) (layer B.Cu) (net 1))
 (segment (start 156.5 109.75) (end 156.5 110.25) (width 0.25) (layer B.Cu) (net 1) (status 800000))
 (segment (start 154 101.25) (end 155.5 101.25) (width 0.25) (layer B.Cu) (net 1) (status 400000))
 (segment (start 156.5 100.25) (end 156.5 99.75) (width 0.25) (layer B.Cu) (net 1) (status 800000))
 (segment (start 155.5 101.25) (end 156.5 100.25) (width 0.25) (layer B.Cu) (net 1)))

